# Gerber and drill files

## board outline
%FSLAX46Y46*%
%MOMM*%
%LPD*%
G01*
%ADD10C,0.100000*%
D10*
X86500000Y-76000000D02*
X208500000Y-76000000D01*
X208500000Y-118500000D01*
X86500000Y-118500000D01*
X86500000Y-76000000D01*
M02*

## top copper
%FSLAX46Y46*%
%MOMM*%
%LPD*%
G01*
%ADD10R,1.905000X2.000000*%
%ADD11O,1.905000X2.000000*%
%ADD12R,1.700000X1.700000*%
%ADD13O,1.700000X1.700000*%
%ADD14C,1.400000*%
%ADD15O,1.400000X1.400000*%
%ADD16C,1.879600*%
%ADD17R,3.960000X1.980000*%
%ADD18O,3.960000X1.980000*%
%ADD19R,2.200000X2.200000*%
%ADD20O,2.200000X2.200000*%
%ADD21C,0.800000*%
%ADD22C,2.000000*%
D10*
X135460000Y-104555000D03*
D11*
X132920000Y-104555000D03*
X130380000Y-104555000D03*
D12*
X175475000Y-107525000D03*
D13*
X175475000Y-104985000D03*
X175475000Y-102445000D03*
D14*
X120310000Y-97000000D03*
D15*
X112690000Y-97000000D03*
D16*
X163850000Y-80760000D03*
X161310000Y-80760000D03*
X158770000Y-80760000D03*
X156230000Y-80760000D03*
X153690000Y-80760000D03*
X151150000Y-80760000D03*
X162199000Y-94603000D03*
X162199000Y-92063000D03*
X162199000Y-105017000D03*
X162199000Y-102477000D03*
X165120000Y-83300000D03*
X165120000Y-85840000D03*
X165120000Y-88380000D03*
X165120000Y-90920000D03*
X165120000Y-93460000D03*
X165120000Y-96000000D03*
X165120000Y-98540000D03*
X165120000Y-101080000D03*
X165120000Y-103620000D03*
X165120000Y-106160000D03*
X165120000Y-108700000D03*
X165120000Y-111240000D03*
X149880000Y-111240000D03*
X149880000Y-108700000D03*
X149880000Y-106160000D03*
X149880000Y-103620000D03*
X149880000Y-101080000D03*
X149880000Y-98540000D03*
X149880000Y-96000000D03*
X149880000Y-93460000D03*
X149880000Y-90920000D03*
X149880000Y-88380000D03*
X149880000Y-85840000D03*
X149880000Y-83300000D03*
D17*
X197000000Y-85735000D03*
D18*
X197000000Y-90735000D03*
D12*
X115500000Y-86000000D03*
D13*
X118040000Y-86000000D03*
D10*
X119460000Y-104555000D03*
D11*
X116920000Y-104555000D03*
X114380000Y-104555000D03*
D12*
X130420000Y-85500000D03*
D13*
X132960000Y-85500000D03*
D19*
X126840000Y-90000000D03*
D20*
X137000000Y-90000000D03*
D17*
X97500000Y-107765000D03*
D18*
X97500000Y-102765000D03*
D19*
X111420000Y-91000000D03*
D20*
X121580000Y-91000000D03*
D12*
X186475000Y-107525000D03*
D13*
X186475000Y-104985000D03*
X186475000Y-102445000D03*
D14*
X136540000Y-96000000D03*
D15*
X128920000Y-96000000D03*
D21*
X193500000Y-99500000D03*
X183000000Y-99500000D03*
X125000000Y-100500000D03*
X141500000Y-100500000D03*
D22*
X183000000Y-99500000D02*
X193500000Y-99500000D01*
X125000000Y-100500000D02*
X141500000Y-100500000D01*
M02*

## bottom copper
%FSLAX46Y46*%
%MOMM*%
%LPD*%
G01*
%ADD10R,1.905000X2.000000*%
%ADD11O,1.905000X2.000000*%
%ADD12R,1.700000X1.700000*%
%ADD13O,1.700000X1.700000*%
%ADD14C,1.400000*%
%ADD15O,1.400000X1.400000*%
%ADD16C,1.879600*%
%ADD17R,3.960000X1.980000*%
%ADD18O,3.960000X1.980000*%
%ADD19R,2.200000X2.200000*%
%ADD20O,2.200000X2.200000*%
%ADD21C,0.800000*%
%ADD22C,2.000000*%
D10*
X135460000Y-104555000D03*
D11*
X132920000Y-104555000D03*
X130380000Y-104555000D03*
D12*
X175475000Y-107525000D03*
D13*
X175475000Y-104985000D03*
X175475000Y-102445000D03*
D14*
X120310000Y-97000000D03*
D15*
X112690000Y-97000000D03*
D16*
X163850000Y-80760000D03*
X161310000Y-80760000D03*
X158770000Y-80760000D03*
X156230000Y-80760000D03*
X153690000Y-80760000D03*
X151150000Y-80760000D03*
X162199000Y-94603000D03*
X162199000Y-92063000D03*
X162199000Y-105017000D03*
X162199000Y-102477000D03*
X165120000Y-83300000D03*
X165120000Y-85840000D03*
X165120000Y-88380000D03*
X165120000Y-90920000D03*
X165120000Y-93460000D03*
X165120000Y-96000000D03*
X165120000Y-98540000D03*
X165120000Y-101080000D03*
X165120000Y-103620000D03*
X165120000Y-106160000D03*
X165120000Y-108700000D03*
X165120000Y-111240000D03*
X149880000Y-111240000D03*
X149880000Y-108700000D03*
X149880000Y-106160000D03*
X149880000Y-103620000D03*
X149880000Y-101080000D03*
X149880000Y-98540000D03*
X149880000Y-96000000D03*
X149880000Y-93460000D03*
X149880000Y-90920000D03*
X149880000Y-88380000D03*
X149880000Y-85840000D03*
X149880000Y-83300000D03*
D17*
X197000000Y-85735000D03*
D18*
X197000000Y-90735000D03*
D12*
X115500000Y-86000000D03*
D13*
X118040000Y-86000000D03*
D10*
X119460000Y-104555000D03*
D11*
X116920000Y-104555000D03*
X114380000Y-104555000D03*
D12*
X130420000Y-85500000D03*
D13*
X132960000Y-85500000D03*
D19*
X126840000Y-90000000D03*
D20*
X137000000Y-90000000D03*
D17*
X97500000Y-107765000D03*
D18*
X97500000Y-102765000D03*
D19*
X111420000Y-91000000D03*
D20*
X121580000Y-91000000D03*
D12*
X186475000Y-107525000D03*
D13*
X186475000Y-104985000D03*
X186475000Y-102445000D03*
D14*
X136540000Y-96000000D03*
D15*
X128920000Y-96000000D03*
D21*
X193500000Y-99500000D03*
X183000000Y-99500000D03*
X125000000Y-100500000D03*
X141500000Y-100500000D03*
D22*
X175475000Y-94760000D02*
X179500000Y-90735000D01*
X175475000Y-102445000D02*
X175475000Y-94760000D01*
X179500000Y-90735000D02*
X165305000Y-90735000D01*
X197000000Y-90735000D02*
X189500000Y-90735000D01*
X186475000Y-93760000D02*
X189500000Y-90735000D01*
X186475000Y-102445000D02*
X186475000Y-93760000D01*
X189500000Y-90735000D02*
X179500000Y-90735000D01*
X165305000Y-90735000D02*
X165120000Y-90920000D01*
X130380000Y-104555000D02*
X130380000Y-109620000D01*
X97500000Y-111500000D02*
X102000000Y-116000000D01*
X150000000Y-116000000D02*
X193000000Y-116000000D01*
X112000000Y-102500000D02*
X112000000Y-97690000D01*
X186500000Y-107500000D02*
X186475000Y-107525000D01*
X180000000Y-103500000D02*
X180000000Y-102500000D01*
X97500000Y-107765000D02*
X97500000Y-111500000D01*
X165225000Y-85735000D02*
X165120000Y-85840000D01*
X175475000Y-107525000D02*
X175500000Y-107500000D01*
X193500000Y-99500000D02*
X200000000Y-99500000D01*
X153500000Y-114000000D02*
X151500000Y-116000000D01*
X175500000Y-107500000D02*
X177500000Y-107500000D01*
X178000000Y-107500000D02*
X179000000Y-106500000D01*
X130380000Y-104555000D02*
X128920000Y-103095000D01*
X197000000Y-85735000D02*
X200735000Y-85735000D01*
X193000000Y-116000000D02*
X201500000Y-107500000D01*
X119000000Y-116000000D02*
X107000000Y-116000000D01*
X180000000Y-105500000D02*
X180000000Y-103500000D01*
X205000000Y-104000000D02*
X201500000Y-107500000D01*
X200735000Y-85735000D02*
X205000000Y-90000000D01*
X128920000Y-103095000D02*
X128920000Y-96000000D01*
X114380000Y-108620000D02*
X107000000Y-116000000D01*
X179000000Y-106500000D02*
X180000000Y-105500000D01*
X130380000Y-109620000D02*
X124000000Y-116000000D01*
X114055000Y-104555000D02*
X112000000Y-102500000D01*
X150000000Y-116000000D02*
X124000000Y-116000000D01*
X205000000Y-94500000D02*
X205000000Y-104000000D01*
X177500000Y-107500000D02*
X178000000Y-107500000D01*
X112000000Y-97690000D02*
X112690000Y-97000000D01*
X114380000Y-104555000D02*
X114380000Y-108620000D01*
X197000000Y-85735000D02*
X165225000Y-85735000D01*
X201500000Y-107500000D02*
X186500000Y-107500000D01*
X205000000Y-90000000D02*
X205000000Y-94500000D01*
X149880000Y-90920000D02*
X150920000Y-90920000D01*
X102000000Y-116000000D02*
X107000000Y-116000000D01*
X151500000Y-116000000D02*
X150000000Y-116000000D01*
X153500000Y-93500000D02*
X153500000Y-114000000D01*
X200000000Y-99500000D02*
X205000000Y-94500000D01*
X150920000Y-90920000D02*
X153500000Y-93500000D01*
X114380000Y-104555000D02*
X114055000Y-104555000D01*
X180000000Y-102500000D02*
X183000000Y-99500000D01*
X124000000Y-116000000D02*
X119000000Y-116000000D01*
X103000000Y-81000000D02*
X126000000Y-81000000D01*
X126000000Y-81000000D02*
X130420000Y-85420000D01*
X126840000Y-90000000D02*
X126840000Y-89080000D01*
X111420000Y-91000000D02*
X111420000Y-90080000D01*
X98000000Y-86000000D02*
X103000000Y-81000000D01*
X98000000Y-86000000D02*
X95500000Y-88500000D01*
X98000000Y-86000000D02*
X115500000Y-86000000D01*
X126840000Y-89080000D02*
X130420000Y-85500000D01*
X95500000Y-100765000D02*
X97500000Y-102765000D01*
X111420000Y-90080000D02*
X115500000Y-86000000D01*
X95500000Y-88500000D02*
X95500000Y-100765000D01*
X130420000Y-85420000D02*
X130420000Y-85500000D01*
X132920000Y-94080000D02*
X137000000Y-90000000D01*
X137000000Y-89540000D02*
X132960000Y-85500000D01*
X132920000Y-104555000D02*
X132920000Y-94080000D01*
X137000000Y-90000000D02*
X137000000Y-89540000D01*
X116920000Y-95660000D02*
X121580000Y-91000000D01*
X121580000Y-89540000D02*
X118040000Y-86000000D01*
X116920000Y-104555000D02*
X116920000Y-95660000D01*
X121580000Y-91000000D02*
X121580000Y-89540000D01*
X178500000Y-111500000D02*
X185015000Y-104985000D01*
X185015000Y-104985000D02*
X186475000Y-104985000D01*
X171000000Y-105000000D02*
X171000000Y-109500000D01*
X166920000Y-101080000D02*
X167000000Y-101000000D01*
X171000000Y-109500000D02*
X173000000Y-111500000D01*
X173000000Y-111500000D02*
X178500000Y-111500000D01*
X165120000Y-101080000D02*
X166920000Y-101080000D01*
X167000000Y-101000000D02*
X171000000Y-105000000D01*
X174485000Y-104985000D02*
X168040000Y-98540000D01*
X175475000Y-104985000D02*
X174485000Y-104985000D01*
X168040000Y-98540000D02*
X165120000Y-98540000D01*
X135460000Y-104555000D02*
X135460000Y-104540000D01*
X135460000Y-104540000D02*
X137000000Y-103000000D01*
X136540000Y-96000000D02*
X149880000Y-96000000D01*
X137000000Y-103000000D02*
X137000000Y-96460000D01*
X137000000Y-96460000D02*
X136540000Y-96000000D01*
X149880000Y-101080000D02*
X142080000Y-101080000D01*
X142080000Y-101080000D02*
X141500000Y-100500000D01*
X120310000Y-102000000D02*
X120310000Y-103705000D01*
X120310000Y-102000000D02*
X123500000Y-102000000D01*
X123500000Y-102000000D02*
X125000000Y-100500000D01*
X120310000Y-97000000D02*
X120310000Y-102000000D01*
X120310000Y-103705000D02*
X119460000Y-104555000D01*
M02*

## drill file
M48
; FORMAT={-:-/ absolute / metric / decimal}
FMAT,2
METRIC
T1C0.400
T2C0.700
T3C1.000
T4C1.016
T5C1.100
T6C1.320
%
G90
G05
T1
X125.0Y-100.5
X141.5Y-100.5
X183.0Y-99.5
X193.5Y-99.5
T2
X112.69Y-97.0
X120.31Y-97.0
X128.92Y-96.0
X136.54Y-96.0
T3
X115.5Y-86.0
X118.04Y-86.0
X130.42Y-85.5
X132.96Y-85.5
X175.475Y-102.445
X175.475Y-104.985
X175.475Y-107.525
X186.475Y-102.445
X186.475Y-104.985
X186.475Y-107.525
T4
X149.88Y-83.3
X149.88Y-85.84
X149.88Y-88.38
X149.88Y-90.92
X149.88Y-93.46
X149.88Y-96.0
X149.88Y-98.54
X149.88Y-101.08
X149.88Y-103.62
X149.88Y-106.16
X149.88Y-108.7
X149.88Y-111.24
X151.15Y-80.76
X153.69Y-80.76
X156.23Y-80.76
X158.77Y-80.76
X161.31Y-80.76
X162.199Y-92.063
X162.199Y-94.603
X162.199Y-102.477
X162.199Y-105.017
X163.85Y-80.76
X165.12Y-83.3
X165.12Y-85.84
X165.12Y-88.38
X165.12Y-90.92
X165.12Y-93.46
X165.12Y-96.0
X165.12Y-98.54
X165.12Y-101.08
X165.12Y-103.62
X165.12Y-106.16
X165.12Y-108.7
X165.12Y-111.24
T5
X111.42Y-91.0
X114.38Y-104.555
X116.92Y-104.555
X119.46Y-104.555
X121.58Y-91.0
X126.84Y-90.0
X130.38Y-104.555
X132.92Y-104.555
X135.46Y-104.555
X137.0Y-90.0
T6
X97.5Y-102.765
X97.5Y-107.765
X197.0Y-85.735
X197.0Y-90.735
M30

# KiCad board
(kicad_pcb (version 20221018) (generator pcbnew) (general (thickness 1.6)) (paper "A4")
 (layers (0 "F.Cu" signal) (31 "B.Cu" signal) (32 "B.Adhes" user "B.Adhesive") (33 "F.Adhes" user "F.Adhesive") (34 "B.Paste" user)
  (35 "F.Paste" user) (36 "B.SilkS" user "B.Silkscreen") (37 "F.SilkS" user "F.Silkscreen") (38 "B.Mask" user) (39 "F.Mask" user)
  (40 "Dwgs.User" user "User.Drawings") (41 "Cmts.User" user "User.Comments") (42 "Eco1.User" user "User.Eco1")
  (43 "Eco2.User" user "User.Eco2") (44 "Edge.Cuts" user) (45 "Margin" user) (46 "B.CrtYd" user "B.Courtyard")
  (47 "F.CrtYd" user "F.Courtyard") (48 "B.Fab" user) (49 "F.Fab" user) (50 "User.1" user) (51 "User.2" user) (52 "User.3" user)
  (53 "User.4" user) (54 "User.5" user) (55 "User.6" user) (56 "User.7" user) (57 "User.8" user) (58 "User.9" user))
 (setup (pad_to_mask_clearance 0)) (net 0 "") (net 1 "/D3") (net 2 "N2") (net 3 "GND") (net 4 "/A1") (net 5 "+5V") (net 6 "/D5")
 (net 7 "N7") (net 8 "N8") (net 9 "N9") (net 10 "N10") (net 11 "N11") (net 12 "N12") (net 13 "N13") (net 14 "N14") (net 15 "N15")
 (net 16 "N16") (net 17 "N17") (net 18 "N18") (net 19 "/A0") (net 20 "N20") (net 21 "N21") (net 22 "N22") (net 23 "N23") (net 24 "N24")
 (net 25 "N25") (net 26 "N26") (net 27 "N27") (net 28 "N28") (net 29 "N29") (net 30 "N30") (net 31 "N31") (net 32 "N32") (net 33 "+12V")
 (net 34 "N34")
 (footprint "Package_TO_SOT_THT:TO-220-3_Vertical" (layer "F.Cu") (at 135.46 104.555 180)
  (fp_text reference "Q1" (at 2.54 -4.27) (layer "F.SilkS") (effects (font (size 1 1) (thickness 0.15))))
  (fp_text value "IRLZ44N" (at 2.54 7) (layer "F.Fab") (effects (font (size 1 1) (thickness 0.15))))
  (pad "1" thru_hole rect (at 0 0 180) (size 1.905 2) (drill 1.1) (layers "*.Cu" "*.Mask") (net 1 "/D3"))
  (pad "2" thru_hole oval (at 2.54 0 180) (size 1.905 2) (drill 1.1) (layers "*.Cu" "*.Mask") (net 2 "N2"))
  (pad "3" thru_hole oval (at 5.08 0 180) (size 1.905 2) (drill 1.1) (layers "*.Cu" "*.Mask") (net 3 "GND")))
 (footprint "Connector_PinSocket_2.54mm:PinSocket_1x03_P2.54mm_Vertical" (layer "F.Cu") (at 175.475 107.525 180)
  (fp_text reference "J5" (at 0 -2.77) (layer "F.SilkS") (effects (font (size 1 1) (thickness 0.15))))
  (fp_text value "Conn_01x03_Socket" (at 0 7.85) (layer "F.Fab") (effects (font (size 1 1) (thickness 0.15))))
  (pad "1" thru_hole rect (at 0 0 180) (size 1.7 1.7) (drill 1) (layers "*.Cu" "*.Mask") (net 3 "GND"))
  (pad "2" thru_hole oval (at 0 2.54 180) (size 1.7 1.7) (drill 1) (layers "*.Cu" "*.Mask") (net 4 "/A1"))
  (pad "3" thru_hole oval (at 0 5.08 180) (size 1.7 1.7) (drill 1) (layers "*.Cu" "*.Mask") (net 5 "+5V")))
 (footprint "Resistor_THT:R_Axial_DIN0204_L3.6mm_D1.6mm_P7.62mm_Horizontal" (layer "F.Cu") (at 120.31 97 180)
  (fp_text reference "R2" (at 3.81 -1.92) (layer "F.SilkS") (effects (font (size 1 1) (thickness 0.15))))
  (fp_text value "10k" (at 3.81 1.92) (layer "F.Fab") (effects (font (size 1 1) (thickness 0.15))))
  (pad "1" thru_hole circle (at 0 0 180) (size 1.4 1.4) (drill 0.7) (layers "*.Cu" "*.Mask") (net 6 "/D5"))
  (pad "2" thru_hole oval (at 7.62 0 180) (size 1.4 1.4) (drill 0.7) (layers "*.Cu" "*.Mask") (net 3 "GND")))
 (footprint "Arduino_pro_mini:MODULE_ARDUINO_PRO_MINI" (layer "F.Cu") (at 157.5 96)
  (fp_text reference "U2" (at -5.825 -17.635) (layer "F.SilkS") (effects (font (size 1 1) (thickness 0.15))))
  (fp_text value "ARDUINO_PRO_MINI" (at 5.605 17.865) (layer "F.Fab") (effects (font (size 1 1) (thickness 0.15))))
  (pad "JP1_1" thru_hole circle (at 6.35 -15.24) (size 1.8796 1.8796) (drill 1.016) (layers "*.Cu" "*.Mask") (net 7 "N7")
   (solder_mask_margin 0.102))
  (pad "JP1_2" thru_hole circle (at 3.81 -15.24) (size 1.8796 1.8796) (drill 1.016) (layers "*.Cu" "*.Mask") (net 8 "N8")
   (solder_mask_margin 0.102))
  (pad "JP1_3" thru_hole circle (at 1.27 -15.24) (size 1.8796 1.8796) (drill 1.016) (layers "*.Cu" "*.Mask") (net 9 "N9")
   (solder_mask_margin 0.102))
  (pad "JP1_4" thru_hole circle (at -1.27 -15.24) (size 1.8796 1.8796) (drill 1.016) (layers "*.Cu" "*.Mask") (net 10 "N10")
   (solder_mask_margin 0.102))
  (pad "JP1_5" thru_hole circle (at -3.81 -15.24) (size 1.8796 1.8796) (drill 1.016) (layers "*.Cu" "*.Mask") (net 3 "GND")
   (solder_mask_margin 0.102))
  (pad "JP1_6" thru_hole circle (at -6.35 -15.24) (size 1.8796 1.8796) (drill 1.016) (layers "*.Cu" "*.Mask") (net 3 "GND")
   (solder_mask_margin 0.102))
  (pad "JP2_1" thru_hole circle (at 4.699 -1.397) (size 1.8796 1.8796) (drill 1.016) (layers "*.Cu" "*.Mask") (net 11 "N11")
   (solder_mask_margin 0.102))
  (pad "JP2_2" thru_hole circle (at 4.699 -3.937) (size 1.8796 1.8796) (drill 1.016) (layers "*.Cu" "*.Mask") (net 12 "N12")
   (solder_mask_margin 0.102))
  (pad "JP3_1" thru_hole circle (at 4.699 9.017) (size 1.8796 1.8796) (drill 1.016) (layers "*.Cu" "*.Mask") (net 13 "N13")
   (solder_mask_margin 0.102))
  (pad "JP3_2" thru_hole circle (at 4.699 6.477) (size 1.8796 1.8796) (drill 1.016) (layers "*.Cu" "*.Mask") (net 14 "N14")
   (solder_mask_margin 0.102))
  (pad "JP6_1" thru_hole circle (at 7.62 -12.7) (size 1.8796 1.8796) (drill 1.016) (layers "*.Cu" "*.Mask") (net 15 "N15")
   (solder_mask_margin 0.102))
  (pad "JP6_2" thru_hole circle (at 7.62 -10.16) (size 1.8796 1.8796) (drill 1.016) (layers "*.Cu" "*.Mask") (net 3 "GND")
   (solder_mask_margin 0.102))
  (pad "JP6_3" thru_hole circle (at 7.62 -7.62) (size 1.8796 1.8796) (drill 1.016) (layers "*.Cu" "*.Mask") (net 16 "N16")
   (solder_mask_margin 0.102))
  (pad "JP6_4" thru_hole circle (at 7.62 -5.08) (size 1.8796 1.8796) (drill 1.016) (layers "*.Cu" "*.Mask") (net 5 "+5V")
   (solder_mask_margin 0.102))
  (pad "JP6_5" thru_hole circle (at 7.62 -2.54) (size 1.8796 1.8796) (drill 1.016) (layers "*.Cu" "*.Mask") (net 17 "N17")
   (solder_mask_margin 0.102))
  (pad "JP6_6" thru_hole circle (at 7.62 0) (size 1.8796 1.8796) (drill 1.016) (layers "*.Cu" "*.Mask") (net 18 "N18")
   (solder_mask_margin 0.102))
  (pad "JP6_7" thru_hole circle (at 7.62 2.54) (size 1.8796 1.8796) (drill 1.016) (layers "*.Cu" "*.Mask") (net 4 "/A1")
   (solder_mask_margin 0.102))
  (pad "JP6_8" thru_hole circle (at 7.62 5.08) (size 1.8796 1.8796) (drill 1.016) (layers "*.Cu" "*.Mask") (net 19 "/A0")
   (solder_mask_margin 0.102))
  (pad "JP6_9" thru_hole circle (at 7.62 7.62) (size 1.8796 1.8796) (drill 1.016) (layers "*.Cu" "*.Mask") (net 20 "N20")
   (solder_mask_margin 0.102))
  (pad "JP6_10" thru_hole circle (at 7.62 10.16) (size 1.8796 1.8796) (drill 1.016) (layers "*.Cu" "*.Mask") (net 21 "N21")
   (solder_mask_margin 0.102))
  (pad "JP6_11" thru_hole circle (at 7.62 12.7) (size 1.8796 1.8796) (drill 1.016) (layers "*.Cu" "*.Mask") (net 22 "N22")
   (solder_mask_margin 0.102))
  (pad "JP6_12" thru_hole circle (at 7.62 15.24) (size 1.8796 1.8796) (drill 1.016) (layers "*.Cu" "*.Mask") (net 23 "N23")
   (solder_mask_margin 0.102))
  (pad "JP7_1" thru_hole circle (at -7.62 15.24) (size 1.8796 1.8796) (drill 1.016) (layers "*.Cu" "*.Mask") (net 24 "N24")
   (solder_mask_margin 0.102))
  (pad "JP7_2" thru_hole circle (at -7.62 12.7) (size 1.8796 1.8796) (drill 1.016) (layers "*.Cu" "*.Mask") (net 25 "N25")
   (solder_mask_margin 0.102))
  (pad "JP7_3" thru_hole circle (at -7.62 10.16) (size 1.8796 1.8796) (drill 1.016) (layers "*.Cu" "*.Mask") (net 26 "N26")
   (solder_mask_margin 0.102))
  (pad "JP7_4" thru_hole circle (at -7.62 7.62) (size 1.8796 1.8796) (drill 1.016) (layers "*.Cu" "*.Mask") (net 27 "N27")
   (solder_mask_margin 0.102))
  (pad "JP7_5" thru_hole circle (at -7.62 5.08) (size 1.8796 1.8796) (drill 1.016) (layers "*.Cu" "*.Mask") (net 6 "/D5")
   (solder_mask_margin 0.102))
  (pad "JP7_6" thru_hole circle (at -7.62 2.54) (size 1.8796 1.8796) (drill 1.016) (layers "*.Cu" "*.Mask") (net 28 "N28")
   (solder_mask_margin 0.102))
  (pad "JP7_7" thru_hole circle (at -7.62 0) (size 1.8796 1.8796) (drill 1.016) (layers "*.Cu" "*.Mask") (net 1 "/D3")
   (solder_mask_margin 0.102))
  (pad "JP7_8" thru_hole circle (at -7.62 -2.54) (size 1.8796 1.8796) (drill 1.016) (layers "*.Cu" "*.Mask") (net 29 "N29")
   (solder_mask_margin 0.102))
  (pad "JP7_9" thru_hole circle (at -7.62 -5.08) (size 1.8796 1.8796) (drill 1.016) (layers "*.Cu" "*.Mask") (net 3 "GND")
   (solder_mask_margin 0.102))
  (pad "JP7_10" thru_hole circle (at -7.62 -7.62) (size 1.8796 1.8796) (drill 1.016) (layers "*.Cu" "*.Mask") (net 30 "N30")
   (solder_mask_margin 0.102))
  (pad "JP7_11" thru_hole circle (at -7.62 -10.16) (size 1.8796 1.8796) (drill 1.016) (layers "*.Cu" "*.Mask") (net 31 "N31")
   (solder_mask_margin 0.102))
  (pad "JP7_12" thru_hole circle (at -7.62 -12.7) (size 1.8796 1.8796) (drill 1.016) (layers "*.Cu" "*.Mask") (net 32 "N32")
   (solder_mask_margin 0.102)))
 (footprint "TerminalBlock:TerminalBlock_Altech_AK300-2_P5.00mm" (layer "F.Cu") (at 197 85.735 -90)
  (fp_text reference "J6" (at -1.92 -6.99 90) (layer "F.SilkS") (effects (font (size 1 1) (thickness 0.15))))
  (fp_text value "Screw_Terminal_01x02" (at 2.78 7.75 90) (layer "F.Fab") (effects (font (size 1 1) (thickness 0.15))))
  (pad "1" thru_hole rect (at 0 0 270) (size 1.98 3.96) (drill 1.32) (layers "*.Cu" "*.Mask") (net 3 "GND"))
  (pad "2" thru_hole oval (at 5 0 270) (size 1.98 3.96) (drill 1.32) (layers "*.Cu" "*.Mask") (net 5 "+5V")))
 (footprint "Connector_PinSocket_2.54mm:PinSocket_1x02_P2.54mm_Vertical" (layer "F.Cu") (at 115.5 86 90)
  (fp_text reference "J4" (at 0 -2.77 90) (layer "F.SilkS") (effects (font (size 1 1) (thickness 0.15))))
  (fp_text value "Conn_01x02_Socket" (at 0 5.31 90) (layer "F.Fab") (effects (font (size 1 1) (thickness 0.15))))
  (pad "1" thru_hole rect (at 0 0 90) (size 1.7 1.7) (drill 1) (layers "*.Cu" "*.Mask") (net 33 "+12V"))
  (pad "2" thru_hole oval (at 0 2.54 90) (size 1.7 1.7) (drill 1) (layers "*.Cu" "*.Mask") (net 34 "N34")))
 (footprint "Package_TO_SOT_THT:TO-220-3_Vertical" (layer "F.Cu") (at 119.46 104.555 180)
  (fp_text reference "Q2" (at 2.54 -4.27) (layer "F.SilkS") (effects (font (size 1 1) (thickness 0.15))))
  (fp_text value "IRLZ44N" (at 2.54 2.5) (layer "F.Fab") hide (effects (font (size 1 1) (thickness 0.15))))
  (pad "1" thru_hole rect (at 0 0 180) (size 1.905 2) (drill 1.1) (layers "*.Cu" "*.Mask") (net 6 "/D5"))
  (pad "2" thru_hole oval (at 2.54 0 180) (size 1.905 2) (drill 1.1) (layers "*.Cu" "*.Mask") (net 34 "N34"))
  (pad "3" thru_hole oval (at 5.08 0 180) (size 1.905 2) (drill 1.1) (layers "*.Cu" "*.Mask") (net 3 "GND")))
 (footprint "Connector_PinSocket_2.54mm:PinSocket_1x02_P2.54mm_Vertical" (layer "F.Cu") (at 130.42 85.5 90)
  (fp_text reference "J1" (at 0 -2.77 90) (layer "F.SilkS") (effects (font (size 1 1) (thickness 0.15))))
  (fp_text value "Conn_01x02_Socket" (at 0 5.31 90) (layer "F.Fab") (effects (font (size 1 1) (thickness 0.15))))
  (pad "1" thru_hole rect (at 0 0 90) (size 1.7 1.7) (drill 1) (layers "*.Cu" "*.Mask") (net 33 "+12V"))
  (pad "2" thru_hole oval (at 0 2.54 90) (size 1.7 1.7) (drill 1) (layers "*.Cu" "*.Mask") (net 2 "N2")))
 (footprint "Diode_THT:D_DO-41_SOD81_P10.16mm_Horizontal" (layer "F.Cu") (at 126.84 90)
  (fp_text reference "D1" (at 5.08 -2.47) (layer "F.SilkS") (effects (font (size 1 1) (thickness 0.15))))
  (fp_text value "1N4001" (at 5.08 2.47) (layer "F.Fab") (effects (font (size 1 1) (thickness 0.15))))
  (pad "1" thru_hole rect (at 0 0) (size 2.2 2.2) (drill 1.1) (layers "*.Cu" "*.Mask") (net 33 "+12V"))
  (pad "2" thru_hole oval (at 10.16 0) (size 2.2 2.2) (drill 1.1) (layers "*.Cu" "*.Mask") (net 2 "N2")))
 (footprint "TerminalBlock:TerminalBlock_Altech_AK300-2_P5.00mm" (layer "F.Cu") (at 97.5 107.765 90)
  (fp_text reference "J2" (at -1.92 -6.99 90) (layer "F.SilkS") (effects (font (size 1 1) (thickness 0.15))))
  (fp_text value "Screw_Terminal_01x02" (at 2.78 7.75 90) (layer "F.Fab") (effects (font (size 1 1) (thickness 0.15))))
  (pad "1" thru_hole rect (at 0 0 90) (size 1.98 3.96) (drill 1.32) (layers "*.Cu" "*.Mask") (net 3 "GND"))
  (pad "2" thru_hole oval (at 5 0 90) (size 1.98 3.96) (drill 1.32) (layers "*.Cu" "*.Mask") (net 33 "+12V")))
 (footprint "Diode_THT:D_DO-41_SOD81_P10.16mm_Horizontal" (layer "F.Cu") (at 111.42 91)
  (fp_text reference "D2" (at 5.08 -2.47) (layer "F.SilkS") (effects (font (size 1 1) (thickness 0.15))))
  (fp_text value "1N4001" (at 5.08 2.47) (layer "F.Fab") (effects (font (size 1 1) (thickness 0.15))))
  (pad "1" thru_hole rect (at 0 0) (size 2.2 2.2) (drill 1.1) (layers "*.Cu" "*.Mask") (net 33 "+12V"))
  (pad "2" thru_hole oval (at 10.16 0) (size 2.2 2.2) (drill 1.1) (layers "*.Cu" "*.Mask") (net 34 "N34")))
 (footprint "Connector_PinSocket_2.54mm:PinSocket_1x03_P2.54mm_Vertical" (layer "F.Cu") (at 186.475 107.525 180)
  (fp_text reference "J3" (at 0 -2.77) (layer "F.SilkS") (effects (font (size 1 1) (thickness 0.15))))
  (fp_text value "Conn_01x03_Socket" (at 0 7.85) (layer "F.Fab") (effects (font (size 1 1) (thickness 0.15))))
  (pad "1" thru_hole rect (at 0 0 180) (size 1.7 1.7) (drill 1) (layers "*.Cu" "*.Mask") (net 3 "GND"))
  (pad "2" thru_hole oval (at 0 2.54 180) (size 1.7 1.7) (drill 1) (layers "*.Cu" "*.Mask") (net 19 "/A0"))
  (pad "3" thru_hole oval (at 0 5.08 180) (size 1.7 1.7) (drill 1) (layers "*.Cu" "*.Mask") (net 5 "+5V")))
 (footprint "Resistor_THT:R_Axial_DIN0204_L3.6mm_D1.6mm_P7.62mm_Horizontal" (layer "F.Cu") (at 136.54 96 180)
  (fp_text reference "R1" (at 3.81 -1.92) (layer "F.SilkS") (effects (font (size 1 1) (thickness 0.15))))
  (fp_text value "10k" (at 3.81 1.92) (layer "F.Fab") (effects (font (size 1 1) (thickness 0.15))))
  (pad "1" thru_hole circle (at 0 0 180) (size 1.4 1.4) (drill 0.7) (layers "*.Cu" "*.Mask") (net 1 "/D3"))
  (pad "2" thru_hole oval (at 7.62 0 180) (size 1.4 1.4) (drill 0.7) (layers "*.Cu" "*.Mask") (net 3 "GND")))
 (gr_rect (start 86.5 76) (end 208.5 118.5) (stroke (width 0.1) (type default)) (fill none) (layer "Edge.Cuts"))
 (segment (start 175.475 94.76) (end 179.5 90.735) (width 2) (layer "B.Cu") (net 5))
 (segment (start 175.475 102.445) (end 175.475 94.76) (width 2) (layer "B.Cu") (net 5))
 (segment (start 179.5 90.735) (end 165.305 90.735) (width 2) (layer "B.Cu") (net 5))
 (segment (start 197 90.735) (end 189.5 90.735) (width 2) (layer "B.Cu") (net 5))
 (segment (start 186.475 93.76) (end 189.5 90.735) (width 2) (layer "B.Cu") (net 5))
 (segment (start 186.475 102.445) (end 186.475 93.76) (width 2) (layer "B.Cu") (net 5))
 (segment (start 189.5 90.735) (end 179.5 90.735) (width 2) (layer "B.Cu") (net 5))
 (segment (start 165.305 90.735) (end 165.12 90.92) (width 2) (layer "B.Cu") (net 5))
 (segment (start 183 99.5) (end 193.5 99.5) (width 2) (layer "F.Cu") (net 3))
 (via (at 193.5 99.5) (size 0.8) (drill 0.4) (layers "F.Cu" "B.Cu") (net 3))
 (via (at 183 99.5) (size 0.8) (drill 0.4) (layers "F.Cu" "B.Cu") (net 3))
 (segment (start 130.38 104.555) (end 130.38 109.62) (width 2) (layer "B.Cu") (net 3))
 (segment (start 97.5 111.5) (end 102 116) (width 2) (layer "B.Cu") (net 3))
 (segment (start 150 116) (end 193 116) (width 2) (layer "B.Cu") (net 3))
 (segment (start 112 102.5) (end 112 97.69) (width 2) (layer "B.Cu") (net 3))
 (segment (start 186.5 107.5) (end 186.475 107.525) (width 2) (layer "B.Cu") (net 3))
 (segment (start 180 103.5) (end 180 102.5) (width 2) (layer "B.Cu") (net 3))
 (segment (start 97.5 107.765) (end 97.5 111.5) (width 2) (layer "B.Cu") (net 3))
 (segment (start 165.225 85.735) (end 165.12 85.84) (width 2) (layer "B.Cu") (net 3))
 (segment (start 175.475 107.525) (end 175.5 107.5) (width 2) (layer "B.Cu") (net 3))
 (segment (start 193.5 99.5) (end 200 99.5) (width 2) (layer "B.Cu") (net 3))
 (segment (start 153.5 114) (end 151.5 116) (width 2) (layer "B.Cu") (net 3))
 (segment (start 175.5 107.5) (end 177.5 107.5) (width 2) (layer "B.Cu") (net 3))
 (segment (start 178 107.5) (end 179 106.5) (width 2) (layer "B.Cu") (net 3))
 (segment (start 130.38 104.555) (end 128.92 103.095) (width 2) (layer "B.Cu") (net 3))
 (segment (start 197 85.735) (end 200.735 85.735) (width 2) (layer "B.Cu") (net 3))
 (segment (start 193 116) (end 201.5 107.5) (width 2) (layer "B.Cu") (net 3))
 (segment (start 119 116) (end 107 116) (width 2) (layer "B.Cu") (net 3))
 (segment (start 180 105.5) (end 180 103.5) (width 2) (layer "B.Cu") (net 3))
 (segment (start 205 104) (end 201.5 107.5) (width 2) (layer "B.Cu") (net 3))
 (segment (start 200.735 85.735) (end 205 90) (width 2) (layer "B.Cu") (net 3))
 (segment (start 128.92 103.095) (end 128.92 96) (width 2) (layer "B.Cu") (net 3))
 (segment (start 114.38 108.62) (end 107 116) (width 2) (layer "B.Cu") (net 3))
 (segment (start 179 106.5) (end 180 105.5) (width 2) (layer "B.Cu") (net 3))
 (segment (start 130.38 109.62) (end 124 116) (width 2) (layer "B.Cu") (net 3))
 (segment (start 114.055 104.555) (end 112 102.5) (width 2) (layer "B.Cu") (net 3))
 (segment (start 150 116) (end 124 116) (width 2) (layer "B.Cu") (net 3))
 (segment (start 205 94.5) (end 205 104) (width 2) (layer "B.Cu") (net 3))
 (segment (start 177.5 107.5) (end 178 107.5) (width 2) (layer "B.Cu") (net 3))
 (segment (start 112 97.69) (end 112.69 97) (width 2) (layer "B.Cu") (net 3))
 (segment (start 114.38 104.555) (end 114.38 108.62) (width 2) (layer "B.Cu") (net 3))
 (segment (start 197 85.735) (end 165.225 85.735) (width 2) (layer "B.Cu") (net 3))
 (segment (start 201.5 107.5) (end 186.5 107.5) (width 2) (layer "B.Cu") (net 3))
 (segment (start 205 90) (end 205 94.5) (width 2) (layer "B.Cu") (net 3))
 (segment (start 149.88 90.92) (end 150.92 90.92) (width 2) (layer "B.Cu") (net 3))
 (segment (start 102 116) (end 107 116) (width 2) (layer "B.Cu") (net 3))
 (segment (start 151.5 116) (end 150 116) (width 2) (layer "B.Cu") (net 3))
 (segment (start 153.5 93.5) (end 153.5 114) (width 2) (layer "B.Cu") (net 3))
 (segment (start 200 99.5) (end 205 94.5) (width 2) (layer "B.Cu") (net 3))
 (segment (start 150.92 90.92) (end 153.5 93.5) (width 2) (layer "B.Cu") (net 3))
 (segment (start 114.38 104.555) (end 114.055 104.555) (width 2) (layer "B.Cu") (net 3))
 (segment (start 180 102.5) (end 183 99.5) (width 2) (layer "B.Cu") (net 3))
 (segment (start 124 116) (end 119 116) (width 2) (layer "B.Cu") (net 3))
 (segment (start 103 81) (end 126 81) (width 2) (layer "B.Cu") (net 33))
 (segment (start 126 81) (end 130.42 85.42) (width 2) (layer "B.Cu") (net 33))
 (segment (start 126.84 90) (end 126.84 89.08) (width 2) (layer "B.Cu") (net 33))
 (segment (start 111.42 91) (end 111.42 90.08) (width 2) (layer "B.Cu") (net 33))
 (segment (start 98 86) (end 103 81) (width 2) (layer "B.Cu") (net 33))
 (segment (start 98 86) (end 95.5 88.5) (width 2) (layer "B.Cu") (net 33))
 (segment (start 98 86) (end 115.5 86) (width 2) (layer "B.Cu") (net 33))
 (segment (start 126.84 89.08) (end 130.42 85.5) (width 2) (layer "B.Cu") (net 33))
 (segment (start 95.5 100.765) (end 97.5 102.765) (width 2) (layer "B.Cu") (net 33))
 (segment (start 111.42 90.08) (end 115.5 86) (width 2) (layer "B.Cu") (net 33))
 (segment (start 95.5 88.5) (end 95.5 100.765) (width 2) (layer "B.Cu") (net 33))
 (segment (start 130.42 85.42) (end 130.42 85.5) (width 2) (layer "B.Cu") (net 33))
 (segment (start 132.92 94.08) (end 137 90) (width 2) (layer "B.Cu") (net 2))
 (segment (start 137 89.54) (end 132.96 85.5) (width 2) (layer "B.Cu") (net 2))
 (segment (start 132.92 104.555) (end 132.92 94.08) (width 2) (layer "B.Cu") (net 2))
 (segment (start 137 90) (end 137 89.54) (width 2) (layer "B.Cu") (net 2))
 (segment (start 116.92 95.66) (end 121.58 91) (width 2) (layer "B.Cu") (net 34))
 (segment (start 121.58 89.54) (end 118.04 86) (width 2) (layer "B.Cu") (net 34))
 (segment (start 116.92 104.555) (end 116.92 95.66) (width 2) (layer "B.Cu") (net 34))
 (segment (start 121.58 91) (end 121.58 89.54) (width 2) (layer "B.Cu") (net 34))
 (segment (start 178.5 111.5) (end 185.015 104.985) (width 2) (layer "B.Cu") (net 19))
 (segment (start 185.015 104.985) (end 186.475 104.985) (width 2) (layer "B.Cu") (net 19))
 (segment (start 171 105) (end 171 109.5) (width 2) (layer "B.Cu") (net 19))
 (segment (start 166.92 101.08) (end 167 101) (width 2) (layer "B.Cu") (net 19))
 (segment (start 171 109.5) (end 173 111.5) (width 2) (layer "B.Cu") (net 19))
 (segment (start 173 111.5) (end 178.5 111.5) (width 2) (layer "B.Cu") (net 19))
 (segment (start 165.12 101.08) (end 166.92 101.08) (width 2) (layer "B.Cu") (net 19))
 (segment (start 167 101) (end 171 105) (width 2) (layer "B.Cu") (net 19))
 (segment (start 174.485 104.985) (end 168.04 98.54) (width 2) (layer "B.Cu") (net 4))
 (segment (start 175.475 104.985) (end 174.485 104.985) (width 2) (layer "B.Cu") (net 4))
 (segment (start 168.04 98.54) (end 165.12 98.54) (width 2) (layer "B.Cu") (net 4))
 (segment (start 135.46 104.555) (end 135.46 104.54) (width 2) (layer "B.Cu") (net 1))
 (segment (start 135.46 104.54) (end 137 103) (width 2) (layer "B.Cu") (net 1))
 (segment (start 136.54 96) (end 149.88 96) (width 2) (layer "B.Cu") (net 1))
 (segment (start 137 103) (end 137 96.46) (width 2) (layer "B.Cu") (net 1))
 (segment (start 137 96.46) (end 136.54 96) (width 2) (layer "B.Cu") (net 1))
 (segment (start 125 100.5) (end 141.5 100.5) (width 2) (layer "F.Cu") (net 6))
 (via (at 125 100.5) (size 0.8) (drill 0.4) (layers "F.Cu" "B.Cu") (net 6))
 (via (at 141.5 100.5) (size 0.8) (drill 0.4) (layers "F.Cu" "B.Cu") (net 6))
 (segment (start 149.88 101.08) (end 142.08 101.08) (width 2) (layer "B.Cu") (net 6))
 (segment (start 142.08 101.08) (end 141.5 100.5) (width 2) (layer "B.Cu") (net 6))
 (segment (start 120.31 102) (end 120.31 103.705) (width 2) (layer "B.Cu") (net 6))
 (segment (start 120.31 102) (end 123.5 102) (width 2) (layer "B.Cu") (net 6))
 (segment (start 123.5 102) (end 125 100.5) (width 2) (layer "B.Cu") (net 6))
 (segment (start 120.31 97) (end 120.31 102) (width 2) (layer "B.Cu") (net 6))
 (segment (start 120.31 103.705) (end 119.46 104.555) (width 2) (layer "B.Cu") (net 6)))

